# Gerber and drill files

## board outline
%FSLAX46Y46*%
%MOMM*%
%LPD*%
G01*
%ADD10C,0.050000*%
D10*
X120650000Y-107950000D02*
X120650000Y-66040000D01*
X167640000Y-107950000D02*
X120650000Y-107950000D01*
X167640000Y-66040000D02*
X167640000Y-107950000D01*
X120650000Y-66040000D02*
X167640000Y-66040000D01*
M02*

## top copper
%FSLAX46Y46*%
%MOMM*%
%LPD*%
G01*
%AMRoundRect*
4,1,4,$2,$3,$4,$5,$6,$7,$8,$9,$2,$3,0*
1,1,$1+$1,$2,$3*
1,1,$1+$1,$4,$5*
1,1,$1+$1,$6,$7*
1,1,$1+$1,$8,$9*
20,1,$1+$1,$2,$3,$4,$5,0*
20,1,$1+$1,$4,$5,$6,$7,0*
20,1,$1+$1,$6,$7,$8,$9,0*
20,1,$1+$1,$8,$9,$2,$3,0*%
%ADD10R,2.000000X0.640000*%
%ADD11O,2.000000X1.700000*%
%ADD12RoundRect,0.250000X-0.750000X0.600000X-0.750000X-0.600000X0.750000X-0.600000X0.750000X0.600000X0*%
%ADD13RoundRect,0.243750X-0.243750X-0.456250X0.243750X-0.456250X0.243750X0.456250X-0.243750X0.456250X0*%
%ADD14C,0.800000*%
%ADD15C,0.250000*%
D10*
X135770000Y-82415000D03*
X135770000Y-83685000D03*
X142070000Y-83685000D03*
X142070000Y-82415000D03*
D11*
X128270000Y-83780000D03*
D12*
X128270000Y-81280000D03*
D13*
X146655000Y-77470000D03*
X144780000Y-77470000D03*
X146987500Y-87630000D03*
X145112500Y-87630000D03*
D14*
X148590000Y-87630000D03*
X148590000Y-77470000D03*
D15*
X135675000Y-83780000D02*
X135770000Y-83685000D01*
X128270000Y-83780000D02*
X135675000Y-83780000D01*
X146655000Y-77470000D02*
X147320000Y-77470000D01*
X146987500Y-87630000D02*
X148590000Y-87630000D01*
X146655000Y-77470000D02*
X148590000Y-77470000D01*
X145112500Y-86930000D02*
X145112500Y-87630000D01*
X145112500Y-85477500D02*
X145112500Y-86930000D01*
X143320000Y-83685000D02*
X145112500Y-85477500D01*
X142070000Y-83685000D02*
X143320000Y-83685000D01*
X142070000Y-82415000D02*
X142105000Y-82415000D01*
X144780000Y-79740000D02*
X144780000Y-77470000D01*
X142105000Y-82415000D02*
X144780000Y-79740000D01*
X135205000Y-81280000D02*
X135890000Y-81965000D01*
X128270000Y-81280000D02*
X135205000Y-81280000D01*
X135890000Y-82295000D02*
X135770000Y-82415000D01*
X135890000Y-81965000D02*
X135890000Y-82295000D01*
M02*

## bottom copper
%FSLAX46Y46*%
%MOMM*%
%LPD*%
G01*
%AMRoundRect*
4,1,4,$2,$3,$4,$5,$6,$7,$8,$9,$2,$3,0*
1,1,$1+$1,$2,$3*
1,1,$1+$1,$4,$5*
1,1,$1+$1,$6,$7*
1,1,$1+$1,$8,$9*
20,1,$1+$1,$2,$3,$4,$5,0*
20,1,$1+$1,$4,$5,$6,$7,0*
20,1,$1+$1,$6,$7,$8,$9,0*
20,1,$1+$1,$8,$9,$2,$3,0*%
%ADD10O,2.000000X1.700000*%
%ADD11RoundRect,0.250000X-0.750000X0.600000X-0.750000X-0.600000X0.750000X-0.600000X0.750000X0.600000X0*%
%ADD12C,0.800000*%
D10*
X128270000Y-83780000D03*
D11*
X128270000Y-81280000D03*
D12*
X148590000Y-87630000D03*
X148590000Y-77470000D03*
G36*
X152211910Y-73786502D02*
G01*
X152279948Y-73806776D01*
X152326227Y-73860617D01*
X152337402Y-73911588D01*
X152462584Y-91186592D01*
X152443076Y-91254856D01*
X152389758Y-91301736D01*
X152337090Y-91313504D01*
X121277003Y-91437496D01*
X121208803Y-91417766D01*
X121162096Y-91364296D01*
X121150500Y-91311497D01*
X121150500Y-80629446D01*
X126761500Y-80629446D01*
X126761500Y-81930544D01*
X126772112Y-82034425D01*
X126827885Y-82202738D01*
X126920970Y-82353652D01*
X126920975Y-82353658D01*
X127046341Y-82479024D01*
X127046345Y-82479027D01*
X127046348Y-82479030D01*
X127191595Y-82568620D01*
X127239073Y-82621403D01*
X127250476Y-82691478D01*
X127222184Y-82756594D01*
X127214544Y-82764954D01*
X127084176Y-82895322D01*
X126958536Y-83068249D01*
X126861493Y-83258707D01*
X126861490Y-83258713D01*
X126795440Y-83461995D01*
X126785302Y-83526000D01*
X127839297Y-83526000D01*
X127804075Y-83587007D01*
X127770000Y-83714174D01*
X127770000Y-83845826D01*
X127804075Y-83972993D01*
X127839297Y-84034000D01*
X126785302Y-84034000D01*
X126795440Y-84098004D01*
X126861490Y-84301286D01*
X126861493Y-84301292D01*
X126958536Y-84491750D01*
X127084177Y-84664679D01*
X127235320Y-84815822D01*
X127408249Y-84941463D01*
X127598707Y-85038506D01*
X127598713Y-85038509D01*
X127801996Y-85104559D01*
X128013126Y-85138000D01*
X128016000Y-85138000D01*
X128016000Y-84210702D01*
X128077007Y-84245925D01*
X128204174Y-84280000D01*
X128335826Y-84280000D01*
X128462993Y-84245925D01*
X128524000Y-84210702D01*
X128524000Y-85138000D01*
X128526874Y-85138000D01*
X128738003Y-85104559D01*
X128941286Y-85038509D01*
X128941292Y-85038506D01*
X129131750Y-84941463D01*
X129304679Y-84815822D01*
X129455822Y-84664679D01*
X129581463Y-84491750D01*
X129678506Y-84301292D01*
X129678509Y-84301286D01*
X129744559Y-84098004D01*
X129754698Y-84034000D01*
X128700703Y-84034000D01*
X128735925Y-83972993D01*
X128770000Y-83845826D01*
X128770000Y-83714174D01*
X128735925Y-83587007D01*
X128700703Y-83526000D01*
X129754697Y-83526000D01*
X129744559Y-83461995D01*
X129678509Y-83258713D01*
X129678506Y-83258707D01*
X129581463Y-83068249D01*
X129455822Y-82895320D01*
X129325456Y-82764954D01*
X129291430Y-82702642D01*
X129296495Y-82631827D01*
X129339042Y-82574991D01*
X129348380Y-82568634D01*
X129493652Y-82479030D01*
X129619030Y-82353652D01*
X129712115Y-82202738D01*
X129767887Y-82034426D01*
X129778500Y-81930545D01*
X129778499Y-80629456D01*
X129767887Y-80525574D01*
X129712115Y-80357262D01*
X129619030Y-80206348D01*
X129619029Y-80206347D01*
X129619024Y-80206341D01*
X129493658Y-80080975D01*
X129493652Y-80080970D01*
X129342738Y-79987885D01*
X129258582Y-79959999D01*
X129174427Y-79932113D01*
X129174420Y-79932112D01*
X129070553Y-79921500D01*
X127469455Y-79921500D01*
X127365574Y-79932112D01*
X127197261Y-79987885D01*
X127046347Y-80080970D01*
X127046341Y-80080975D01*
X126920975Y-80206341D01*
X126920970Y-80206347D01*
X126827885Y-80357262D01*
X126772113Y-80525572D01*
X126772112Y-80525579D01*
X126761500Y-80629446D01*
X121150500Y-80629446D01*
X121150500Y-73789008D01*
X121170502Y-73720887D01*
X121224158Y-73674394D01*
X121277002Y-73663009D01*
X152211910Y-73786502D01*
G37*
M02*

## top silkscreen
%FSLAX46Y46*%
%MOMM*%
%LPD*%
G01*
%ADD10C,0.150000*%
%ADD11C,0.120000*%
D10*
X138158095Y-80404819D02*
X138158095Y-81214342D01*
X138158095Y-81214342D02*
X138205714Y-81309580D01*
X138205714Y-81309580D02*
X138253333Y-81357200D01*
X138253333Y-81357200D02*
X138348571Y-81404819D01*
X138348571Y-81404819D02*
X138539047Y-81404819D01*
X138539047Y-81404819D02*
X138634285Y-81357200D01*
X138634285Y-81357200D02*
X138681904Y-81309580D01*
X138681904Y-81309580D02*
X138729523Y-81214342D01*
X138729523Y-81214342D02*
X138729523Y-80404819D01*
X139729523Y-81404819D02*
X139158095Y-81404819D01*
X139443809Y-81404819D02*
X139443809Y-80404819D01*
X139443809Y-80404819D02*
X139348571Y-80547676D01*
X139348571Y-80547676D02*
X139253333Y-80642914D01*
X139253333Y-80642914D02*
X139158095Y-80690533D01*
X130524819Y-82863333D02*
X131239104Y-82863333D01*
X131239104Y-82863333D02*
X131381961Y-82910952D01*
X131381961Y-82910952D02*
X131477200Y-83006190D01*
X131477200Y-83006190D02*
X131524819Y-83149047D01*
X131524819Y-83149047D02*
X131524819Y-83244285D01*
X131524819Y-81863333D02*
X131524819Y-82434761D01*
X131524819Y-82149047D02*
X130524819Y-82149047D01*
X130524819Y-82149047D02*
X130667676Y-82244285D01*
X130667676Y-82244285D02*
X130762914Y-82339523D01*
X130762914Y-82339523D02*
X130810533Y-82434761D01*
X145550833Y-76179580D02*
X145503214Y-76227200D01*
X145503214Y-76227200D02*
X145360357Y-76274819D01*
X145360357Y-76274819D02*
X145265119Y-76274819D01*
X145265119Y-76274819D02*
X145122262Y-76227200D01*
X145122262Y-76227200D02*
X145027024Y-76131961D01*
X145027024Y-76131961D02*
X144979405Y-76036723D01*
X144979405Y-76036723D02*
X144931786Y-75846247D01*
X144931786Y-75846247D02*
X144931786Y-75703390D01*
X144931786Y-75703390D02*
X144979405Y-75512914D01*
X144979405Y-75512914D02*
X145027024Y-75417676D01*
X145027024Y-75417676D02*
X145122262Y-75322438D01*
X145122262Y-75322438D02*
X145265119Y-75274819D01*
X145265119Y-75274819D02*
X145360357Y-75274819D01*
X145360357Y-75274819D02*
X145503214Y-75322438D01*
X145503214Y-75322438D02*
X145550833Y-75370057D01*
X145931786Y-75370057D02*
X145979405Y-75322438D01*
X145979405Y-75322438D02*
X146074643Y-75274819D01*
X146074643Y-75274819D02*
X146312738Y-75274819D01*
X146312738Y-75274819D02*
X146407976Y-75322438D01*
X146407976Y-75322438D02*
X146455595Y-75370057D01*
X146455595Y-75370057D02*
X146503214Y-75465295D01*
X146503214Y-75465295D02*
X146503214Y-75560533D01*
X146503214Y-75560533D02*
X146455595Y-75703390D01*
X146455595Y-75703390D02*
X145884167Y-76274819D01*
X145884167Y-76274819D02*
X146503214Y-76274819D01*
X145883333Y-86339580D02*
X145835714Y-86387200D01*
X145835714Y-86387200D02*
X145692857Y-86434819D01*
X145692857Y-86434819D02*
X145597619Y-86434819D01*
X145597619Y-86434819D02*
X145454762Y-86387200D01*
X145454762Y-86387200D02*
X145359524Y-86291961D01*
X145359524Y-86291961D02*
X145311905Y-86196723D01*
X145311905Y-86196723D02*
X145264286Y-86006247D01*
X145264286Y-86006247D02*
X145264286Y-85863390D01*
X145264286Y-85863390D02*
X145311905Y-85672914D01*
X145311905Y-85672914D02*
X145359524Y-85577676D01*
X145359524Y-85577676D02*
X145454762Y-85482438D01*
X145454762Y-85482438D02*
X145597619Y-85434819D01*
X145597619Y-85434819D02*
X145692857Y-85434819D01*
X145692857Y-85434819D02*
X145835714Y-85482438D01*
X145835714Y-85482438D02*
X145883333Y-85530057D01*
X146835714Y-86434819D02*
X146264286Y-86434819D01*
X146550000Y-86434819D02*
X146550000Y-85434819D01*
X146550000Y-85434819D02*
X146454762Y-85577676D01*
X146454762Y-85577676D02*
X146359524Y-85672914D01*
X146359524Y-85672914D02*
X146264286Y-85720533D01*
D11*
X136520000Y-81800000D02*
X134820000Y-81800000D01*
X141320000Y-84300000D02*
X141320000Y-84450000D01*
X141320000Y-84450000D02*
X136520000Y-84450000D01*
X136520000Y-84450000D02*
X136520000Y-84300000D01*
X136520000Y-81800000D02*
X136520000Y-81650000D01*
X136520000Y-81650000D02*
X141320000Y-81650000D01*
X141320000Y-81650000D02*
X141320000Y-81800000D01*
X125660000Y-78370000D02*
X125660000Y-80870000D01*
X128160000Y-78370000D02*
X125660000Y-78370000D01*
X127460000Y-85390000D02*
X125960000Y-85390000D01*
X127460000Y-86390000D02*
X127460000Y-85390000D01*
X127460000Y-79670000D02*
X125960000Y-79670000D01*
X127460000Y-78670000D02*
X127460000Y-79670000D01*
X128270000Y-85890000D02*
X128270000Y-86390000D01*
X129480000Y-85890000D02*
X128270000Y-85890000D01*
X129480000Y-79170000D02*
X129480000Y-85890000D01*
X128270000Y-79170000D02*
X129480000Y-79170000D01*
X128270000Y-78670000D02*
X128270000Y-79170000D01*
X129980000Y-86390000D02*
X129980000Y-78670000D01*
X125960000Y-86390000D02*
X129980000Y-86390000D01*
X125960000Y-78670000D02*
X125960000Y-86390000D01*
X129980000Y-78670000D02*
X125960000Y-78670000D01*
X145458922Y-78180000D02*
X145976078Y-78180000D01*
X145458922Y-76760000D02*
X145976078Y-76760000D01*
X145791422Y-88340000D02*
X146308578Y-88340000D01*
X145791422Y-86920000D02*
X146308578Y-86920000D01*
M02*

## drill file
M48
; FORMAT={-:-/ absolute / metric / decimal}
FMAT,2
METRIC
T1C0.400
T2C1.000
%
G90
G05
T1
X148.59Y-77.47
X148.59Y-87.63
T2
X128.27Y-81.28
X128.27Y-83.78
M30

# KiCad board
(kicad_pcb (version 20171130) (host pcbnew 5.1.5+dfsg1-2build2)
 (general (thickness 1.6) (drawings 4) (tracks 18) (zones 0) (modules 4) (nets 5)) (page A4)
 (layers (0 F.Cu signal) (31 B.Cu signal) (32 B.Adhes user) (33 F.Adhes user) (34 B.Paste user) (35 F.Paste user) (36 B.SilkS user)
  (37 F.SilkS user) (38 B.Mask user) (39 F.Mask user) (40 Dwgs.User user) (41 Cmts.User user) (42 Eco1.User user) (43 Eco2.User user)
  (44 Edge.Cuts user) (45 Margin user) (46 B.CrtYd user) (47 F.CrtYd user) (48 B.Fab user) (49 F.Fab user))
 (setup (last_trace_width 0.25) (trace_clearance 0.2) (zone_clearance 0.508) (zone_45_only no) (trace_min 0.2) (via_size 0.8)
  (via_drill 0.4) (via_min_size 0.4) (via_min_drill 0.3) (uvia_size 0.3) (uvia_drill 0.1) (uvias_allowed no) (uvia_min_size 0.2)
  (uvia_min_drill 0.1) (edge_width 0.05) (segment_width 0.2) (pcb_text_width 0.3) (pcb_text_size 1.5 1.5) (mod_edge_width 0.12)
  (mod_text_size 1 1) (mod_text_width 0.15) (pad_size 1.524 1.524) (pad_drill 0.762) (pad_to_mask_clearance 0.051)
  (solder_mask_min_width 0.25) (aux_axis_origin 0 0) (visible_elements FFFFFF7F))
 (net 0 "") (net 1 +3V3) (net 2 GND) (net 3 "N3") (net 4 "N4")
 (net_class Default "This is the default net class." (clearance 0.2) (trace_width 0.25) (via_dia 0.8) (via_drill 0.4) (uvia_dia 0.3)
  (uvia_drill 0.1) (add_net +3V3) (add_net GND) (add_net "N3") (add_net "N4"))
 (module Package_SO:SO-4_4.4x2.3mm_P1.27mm (layer F.Cu) (at 138.92 83.05)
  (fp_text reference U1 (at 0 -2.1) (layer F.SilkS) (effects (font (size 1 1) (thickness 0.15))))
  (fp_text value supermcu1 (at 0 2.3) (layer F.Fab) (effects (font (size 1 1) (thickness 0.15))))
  (fp_line (start -2.4 -1.25) (end -4.1 -1.25) (layer F.SilkS) (width 0.12))
  (fp_line (start 2.4 1.25) (end 2.4 1.4) (layer F.SilkS) (width 0.12))
  (fp_line (start 2.4 1.4) (end -2.4 1.4) (layer F.SilkS) (width 0.12))
  (fp_line (start -2.4 1.4) (end -2.4 1.25) (layer F.SilkS) (width 0.12))
  (fp_line (start -2.4 -1.25) (end -2.4 -1.4) (layer F.SilkS) (width 0.12))
  (fp_line (start -2.4 -1.4) (end 2.4 -1.4) (layer F.SilkS) (width 0.12))
  (fp_line (start 2.4 -1.4) (end 2.4 -1.25) (layer F.SilkS) (width 0.12))
  (pad 1 smd rect (at -3.15 -0.635) (size 2 0.64) (layers F.Cu F.Paste F.Mask) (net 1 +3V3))
  (pad 2 smd rect (at -3.15 0.635) (size 2 0.64) (layers F.Cu F.Paste F.Mask) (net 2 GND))
  (pad 3 smd rect (at 3.15 0.635) (size 2 0.64) (layers F.Cu F.Paste F.Mask) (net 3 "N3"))
  (pad 4 smd rect (at 3.15 -0.635) (size 2 0.64) (layers F.Cu F.Paste F.Mask) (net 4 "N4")))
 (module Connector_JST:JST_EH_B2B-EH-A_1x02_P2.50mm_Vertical (layer F.Cu) (at 128.27 81.28 270)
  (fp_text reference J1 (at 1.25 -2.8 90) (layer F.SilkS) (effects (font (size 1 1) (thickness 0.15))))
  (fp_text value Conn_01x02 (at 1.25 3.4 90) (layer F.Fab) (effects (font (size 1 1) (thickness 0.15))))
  (fp_line (start -2.91 2.61) (end -0.41 2.61) (layer F.SilkS) (width 0.12))
  (fp_line (start -2.91 0.11) (end -2.91 2.61) (layer F.SilkS) (width 0.12))
  (fp_line (start 4.11 0.81) (end 4.11 2.31) (layer F.SilkS) (width 0.12))
  (fp_line (start 5.11 0.81) (end 4.11 0.81) (layer F.SilkS) (width 0.12))
  (fp_line (start -1.61 0.81) (end -1.61 2.31) (layer F.SilkS) (width 0.12))
  (fp_line (start -2.61 0.81) (end -1.61 0.81) (layer F.SilkS) (width 0.12))
  (fp_line (start 4.61 0) (end 5.11 0) (layer F.SilkS) (width 0.12))
  (fp_line (start 4.61 -1.21) (end 4.61 0) (layer F.SilkS) (width 0.12))
  (fp_line (start -2.11 -1.21) (end 4.61 -1.21) (layer F.SilkS) (width 0.12))
  (fp_line (start -2.11 0) (end -2.11 -1.21) (layer F.SilkS) (width 0.12))
  (fp_line (start -2.61 0) (end -2.11 0) (layer F.SilkS) (width 0.12))
  (fp_line (start 5.11 -1.71) (end -2.61 -1.71) (layer F.SilkS) (width 0.12))
  (fp_line (start 5.11 2.31) (end 5.11 -1.71) (layer F.SilkS) (width 0.12))
  (fp_line (start -2.61 2.31) (end 5.11 2.31) (layer F.SilkS) (width 0.12))
  (fp_line (start -2.61 -1.71) (end -2.61 2.31) (layer F.SilkS) (width 0.12))
  (pad 2 thru_hole oval (at 2.5 0 270) (size 1.7 2) (drill 1) (layers *.Cu *.Mask) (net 2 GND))
  (pad 1 thru_hole roundrect (at 0 0 270) (size 1.7 2) (drill 1) (layers *.Cu *.Mask) (roundrect_rratio 0.147059) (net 1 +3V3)))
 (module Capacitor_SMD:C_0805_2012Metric (layer F.Cu) (at 145.7175 77.47)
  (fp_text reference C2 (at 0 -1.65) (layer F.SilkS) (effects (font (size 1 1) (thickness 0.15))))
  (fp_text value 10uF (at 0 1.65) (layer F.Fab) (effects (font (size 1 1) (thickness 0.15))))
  (fp_line (start -0.258578 0.71) (end 0.258578 0.71) (layer F.SilkS) (width 0.12))
  (fp_line (start -0.258578 -0.71) (end 0.258578 -0.71) (layer F.SilkS) (width 0.12))
  (pad 2 smd roundrect (at 0.9375 0) (size 0.975 1.4) (layers F.Cu F.Paste F.Mask) (roundrect_rratio 0.25) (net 2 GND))
  (pad 1 smd roundrect (at -0.9375 0) (size 0.975 1.4) (layers F.Cu F.Paste F.Mask) (roundrect_rratio 0.25) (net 4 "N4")))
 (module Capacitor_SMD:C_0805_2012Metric (layer F.Cu) (at 146.05 87.63)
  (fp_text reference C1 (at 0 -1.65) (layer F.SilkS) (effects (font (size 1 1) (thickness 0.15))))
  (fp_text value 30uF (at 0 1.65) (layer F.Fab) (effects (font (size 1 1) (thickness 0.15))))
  (fp_line (start -0.258578 0.71) (end 0.258578 0.71) (layer F.SilkS) (width 0.12))
  (fp_line (start -0.258578 -0.71) (end 0.258578 -0.71) (layer F.SilkS) (width 0.12))
  (pad 2 smd roundrect (at 0.9375 0) (size 0.975 1.4) (layers F.Cu F.Paste F.Mask) (roundrect_rratio 0.25) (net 2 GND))
  (pad 1 smd roundrect (at -0.9375 0) (size 0.975 1.4) (layers F.Cu F.Paste F.Mask) (roundrect_rratio 0.25) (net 3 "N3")))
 (gr_line (start 120.65 107.95) (end 120.65 66.04) (layer Edge.Cuts) (width 0.05))
 (gr_line (start 167.64 107.95) (end 120.65 107.95) (layer Edge.Cuts) (width 0.05))
 (gr_line (start 167.64 66.04) (end 167.64 107.95) (layer Edge.Cuts) (width 0.05))
 (gr_line (start 120.65 66.04) (end 167.64 66.04) (layer Edge.Cuts) (width 0.05))
 (segment (start 135.675 83.78) (end 135.77 83.685) (width 0.25) (layer F.Cu) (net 2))
 (segment (start 128.27 83.78) (end 135.675 83.78) (width 0.25) (layer F.Cu) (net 2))
 (segment (start 146.655 77.47) (end 147.32 77.47) (width 0.25) (layer F.Cu) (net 2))
 (via (at 148.59 87.63) (size 0.8) (drill 0.4) (layers F.Cu B.Cu) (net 2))
 (segment (start 146.9875 87.63) (end 148.59 87.63) (width 0.25) (layer F.Cu) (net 2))
 (via (at 148.59 77.47) (size 0.8) (drill 0.4) (layers F.Cu B.Cu) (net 2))
 (segment (start 146.655 77.47) (end 148.59 77.47) (width 0.25) (layer F.Cu) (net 2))
 (segment (start 145.1125 86.93) (end 145.1125 87.63) (width 0.25) (layer F.Cu) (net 3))
 (segment (start 145.1125 85.4775) (end 145.1125 86.93) (width 0.25) (layer F.Cu) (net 3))
 (segment (start 143.32 83.685) (end 145.1125 85.4775) (width 0.25) (layer F.Cu) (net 3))
 (segment (start 142.07 83.685) (end 143.32 83.685) (width 0.25) (layer F.Cu) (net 3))
 (segment (start 142.07 82.415) (end 142.105 82.415) (width 0.25) (layer F.Cu) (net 4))
 (segment (start 144.78 79.74) (end 144.78 77.47) (width 0.25) (layer F.Cu) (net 4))
 (segment (start 142.105 82.415) (end 144.78 79.74) (width 0.25) (layer F.Cu) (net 4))
 (segment (start 135.205 81.28) (end 135.89 81.965) (width 0.25) (layer F.Cu) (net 1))
 (segment (start 128.27 81.28) (end 135.205 81.28) (width 0.25) (layer F.Cu) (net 1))
 (segment (start 135.89 82.295) (end 135.77 82.415) (width 0.25) (layer F.Cu) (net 1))
 (segment (start 135.89 81.965) (end 135.89 82.295) (width 0.25) (layer F.Cu) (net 1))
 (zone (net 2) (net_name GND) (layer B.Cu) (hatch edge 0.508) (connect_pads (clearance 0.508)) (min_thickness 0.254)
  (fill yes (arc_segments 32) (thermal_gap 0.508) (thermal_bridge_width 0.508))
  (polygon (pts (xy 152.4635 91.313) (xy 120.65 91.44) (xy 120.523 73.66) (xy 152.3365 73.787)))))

